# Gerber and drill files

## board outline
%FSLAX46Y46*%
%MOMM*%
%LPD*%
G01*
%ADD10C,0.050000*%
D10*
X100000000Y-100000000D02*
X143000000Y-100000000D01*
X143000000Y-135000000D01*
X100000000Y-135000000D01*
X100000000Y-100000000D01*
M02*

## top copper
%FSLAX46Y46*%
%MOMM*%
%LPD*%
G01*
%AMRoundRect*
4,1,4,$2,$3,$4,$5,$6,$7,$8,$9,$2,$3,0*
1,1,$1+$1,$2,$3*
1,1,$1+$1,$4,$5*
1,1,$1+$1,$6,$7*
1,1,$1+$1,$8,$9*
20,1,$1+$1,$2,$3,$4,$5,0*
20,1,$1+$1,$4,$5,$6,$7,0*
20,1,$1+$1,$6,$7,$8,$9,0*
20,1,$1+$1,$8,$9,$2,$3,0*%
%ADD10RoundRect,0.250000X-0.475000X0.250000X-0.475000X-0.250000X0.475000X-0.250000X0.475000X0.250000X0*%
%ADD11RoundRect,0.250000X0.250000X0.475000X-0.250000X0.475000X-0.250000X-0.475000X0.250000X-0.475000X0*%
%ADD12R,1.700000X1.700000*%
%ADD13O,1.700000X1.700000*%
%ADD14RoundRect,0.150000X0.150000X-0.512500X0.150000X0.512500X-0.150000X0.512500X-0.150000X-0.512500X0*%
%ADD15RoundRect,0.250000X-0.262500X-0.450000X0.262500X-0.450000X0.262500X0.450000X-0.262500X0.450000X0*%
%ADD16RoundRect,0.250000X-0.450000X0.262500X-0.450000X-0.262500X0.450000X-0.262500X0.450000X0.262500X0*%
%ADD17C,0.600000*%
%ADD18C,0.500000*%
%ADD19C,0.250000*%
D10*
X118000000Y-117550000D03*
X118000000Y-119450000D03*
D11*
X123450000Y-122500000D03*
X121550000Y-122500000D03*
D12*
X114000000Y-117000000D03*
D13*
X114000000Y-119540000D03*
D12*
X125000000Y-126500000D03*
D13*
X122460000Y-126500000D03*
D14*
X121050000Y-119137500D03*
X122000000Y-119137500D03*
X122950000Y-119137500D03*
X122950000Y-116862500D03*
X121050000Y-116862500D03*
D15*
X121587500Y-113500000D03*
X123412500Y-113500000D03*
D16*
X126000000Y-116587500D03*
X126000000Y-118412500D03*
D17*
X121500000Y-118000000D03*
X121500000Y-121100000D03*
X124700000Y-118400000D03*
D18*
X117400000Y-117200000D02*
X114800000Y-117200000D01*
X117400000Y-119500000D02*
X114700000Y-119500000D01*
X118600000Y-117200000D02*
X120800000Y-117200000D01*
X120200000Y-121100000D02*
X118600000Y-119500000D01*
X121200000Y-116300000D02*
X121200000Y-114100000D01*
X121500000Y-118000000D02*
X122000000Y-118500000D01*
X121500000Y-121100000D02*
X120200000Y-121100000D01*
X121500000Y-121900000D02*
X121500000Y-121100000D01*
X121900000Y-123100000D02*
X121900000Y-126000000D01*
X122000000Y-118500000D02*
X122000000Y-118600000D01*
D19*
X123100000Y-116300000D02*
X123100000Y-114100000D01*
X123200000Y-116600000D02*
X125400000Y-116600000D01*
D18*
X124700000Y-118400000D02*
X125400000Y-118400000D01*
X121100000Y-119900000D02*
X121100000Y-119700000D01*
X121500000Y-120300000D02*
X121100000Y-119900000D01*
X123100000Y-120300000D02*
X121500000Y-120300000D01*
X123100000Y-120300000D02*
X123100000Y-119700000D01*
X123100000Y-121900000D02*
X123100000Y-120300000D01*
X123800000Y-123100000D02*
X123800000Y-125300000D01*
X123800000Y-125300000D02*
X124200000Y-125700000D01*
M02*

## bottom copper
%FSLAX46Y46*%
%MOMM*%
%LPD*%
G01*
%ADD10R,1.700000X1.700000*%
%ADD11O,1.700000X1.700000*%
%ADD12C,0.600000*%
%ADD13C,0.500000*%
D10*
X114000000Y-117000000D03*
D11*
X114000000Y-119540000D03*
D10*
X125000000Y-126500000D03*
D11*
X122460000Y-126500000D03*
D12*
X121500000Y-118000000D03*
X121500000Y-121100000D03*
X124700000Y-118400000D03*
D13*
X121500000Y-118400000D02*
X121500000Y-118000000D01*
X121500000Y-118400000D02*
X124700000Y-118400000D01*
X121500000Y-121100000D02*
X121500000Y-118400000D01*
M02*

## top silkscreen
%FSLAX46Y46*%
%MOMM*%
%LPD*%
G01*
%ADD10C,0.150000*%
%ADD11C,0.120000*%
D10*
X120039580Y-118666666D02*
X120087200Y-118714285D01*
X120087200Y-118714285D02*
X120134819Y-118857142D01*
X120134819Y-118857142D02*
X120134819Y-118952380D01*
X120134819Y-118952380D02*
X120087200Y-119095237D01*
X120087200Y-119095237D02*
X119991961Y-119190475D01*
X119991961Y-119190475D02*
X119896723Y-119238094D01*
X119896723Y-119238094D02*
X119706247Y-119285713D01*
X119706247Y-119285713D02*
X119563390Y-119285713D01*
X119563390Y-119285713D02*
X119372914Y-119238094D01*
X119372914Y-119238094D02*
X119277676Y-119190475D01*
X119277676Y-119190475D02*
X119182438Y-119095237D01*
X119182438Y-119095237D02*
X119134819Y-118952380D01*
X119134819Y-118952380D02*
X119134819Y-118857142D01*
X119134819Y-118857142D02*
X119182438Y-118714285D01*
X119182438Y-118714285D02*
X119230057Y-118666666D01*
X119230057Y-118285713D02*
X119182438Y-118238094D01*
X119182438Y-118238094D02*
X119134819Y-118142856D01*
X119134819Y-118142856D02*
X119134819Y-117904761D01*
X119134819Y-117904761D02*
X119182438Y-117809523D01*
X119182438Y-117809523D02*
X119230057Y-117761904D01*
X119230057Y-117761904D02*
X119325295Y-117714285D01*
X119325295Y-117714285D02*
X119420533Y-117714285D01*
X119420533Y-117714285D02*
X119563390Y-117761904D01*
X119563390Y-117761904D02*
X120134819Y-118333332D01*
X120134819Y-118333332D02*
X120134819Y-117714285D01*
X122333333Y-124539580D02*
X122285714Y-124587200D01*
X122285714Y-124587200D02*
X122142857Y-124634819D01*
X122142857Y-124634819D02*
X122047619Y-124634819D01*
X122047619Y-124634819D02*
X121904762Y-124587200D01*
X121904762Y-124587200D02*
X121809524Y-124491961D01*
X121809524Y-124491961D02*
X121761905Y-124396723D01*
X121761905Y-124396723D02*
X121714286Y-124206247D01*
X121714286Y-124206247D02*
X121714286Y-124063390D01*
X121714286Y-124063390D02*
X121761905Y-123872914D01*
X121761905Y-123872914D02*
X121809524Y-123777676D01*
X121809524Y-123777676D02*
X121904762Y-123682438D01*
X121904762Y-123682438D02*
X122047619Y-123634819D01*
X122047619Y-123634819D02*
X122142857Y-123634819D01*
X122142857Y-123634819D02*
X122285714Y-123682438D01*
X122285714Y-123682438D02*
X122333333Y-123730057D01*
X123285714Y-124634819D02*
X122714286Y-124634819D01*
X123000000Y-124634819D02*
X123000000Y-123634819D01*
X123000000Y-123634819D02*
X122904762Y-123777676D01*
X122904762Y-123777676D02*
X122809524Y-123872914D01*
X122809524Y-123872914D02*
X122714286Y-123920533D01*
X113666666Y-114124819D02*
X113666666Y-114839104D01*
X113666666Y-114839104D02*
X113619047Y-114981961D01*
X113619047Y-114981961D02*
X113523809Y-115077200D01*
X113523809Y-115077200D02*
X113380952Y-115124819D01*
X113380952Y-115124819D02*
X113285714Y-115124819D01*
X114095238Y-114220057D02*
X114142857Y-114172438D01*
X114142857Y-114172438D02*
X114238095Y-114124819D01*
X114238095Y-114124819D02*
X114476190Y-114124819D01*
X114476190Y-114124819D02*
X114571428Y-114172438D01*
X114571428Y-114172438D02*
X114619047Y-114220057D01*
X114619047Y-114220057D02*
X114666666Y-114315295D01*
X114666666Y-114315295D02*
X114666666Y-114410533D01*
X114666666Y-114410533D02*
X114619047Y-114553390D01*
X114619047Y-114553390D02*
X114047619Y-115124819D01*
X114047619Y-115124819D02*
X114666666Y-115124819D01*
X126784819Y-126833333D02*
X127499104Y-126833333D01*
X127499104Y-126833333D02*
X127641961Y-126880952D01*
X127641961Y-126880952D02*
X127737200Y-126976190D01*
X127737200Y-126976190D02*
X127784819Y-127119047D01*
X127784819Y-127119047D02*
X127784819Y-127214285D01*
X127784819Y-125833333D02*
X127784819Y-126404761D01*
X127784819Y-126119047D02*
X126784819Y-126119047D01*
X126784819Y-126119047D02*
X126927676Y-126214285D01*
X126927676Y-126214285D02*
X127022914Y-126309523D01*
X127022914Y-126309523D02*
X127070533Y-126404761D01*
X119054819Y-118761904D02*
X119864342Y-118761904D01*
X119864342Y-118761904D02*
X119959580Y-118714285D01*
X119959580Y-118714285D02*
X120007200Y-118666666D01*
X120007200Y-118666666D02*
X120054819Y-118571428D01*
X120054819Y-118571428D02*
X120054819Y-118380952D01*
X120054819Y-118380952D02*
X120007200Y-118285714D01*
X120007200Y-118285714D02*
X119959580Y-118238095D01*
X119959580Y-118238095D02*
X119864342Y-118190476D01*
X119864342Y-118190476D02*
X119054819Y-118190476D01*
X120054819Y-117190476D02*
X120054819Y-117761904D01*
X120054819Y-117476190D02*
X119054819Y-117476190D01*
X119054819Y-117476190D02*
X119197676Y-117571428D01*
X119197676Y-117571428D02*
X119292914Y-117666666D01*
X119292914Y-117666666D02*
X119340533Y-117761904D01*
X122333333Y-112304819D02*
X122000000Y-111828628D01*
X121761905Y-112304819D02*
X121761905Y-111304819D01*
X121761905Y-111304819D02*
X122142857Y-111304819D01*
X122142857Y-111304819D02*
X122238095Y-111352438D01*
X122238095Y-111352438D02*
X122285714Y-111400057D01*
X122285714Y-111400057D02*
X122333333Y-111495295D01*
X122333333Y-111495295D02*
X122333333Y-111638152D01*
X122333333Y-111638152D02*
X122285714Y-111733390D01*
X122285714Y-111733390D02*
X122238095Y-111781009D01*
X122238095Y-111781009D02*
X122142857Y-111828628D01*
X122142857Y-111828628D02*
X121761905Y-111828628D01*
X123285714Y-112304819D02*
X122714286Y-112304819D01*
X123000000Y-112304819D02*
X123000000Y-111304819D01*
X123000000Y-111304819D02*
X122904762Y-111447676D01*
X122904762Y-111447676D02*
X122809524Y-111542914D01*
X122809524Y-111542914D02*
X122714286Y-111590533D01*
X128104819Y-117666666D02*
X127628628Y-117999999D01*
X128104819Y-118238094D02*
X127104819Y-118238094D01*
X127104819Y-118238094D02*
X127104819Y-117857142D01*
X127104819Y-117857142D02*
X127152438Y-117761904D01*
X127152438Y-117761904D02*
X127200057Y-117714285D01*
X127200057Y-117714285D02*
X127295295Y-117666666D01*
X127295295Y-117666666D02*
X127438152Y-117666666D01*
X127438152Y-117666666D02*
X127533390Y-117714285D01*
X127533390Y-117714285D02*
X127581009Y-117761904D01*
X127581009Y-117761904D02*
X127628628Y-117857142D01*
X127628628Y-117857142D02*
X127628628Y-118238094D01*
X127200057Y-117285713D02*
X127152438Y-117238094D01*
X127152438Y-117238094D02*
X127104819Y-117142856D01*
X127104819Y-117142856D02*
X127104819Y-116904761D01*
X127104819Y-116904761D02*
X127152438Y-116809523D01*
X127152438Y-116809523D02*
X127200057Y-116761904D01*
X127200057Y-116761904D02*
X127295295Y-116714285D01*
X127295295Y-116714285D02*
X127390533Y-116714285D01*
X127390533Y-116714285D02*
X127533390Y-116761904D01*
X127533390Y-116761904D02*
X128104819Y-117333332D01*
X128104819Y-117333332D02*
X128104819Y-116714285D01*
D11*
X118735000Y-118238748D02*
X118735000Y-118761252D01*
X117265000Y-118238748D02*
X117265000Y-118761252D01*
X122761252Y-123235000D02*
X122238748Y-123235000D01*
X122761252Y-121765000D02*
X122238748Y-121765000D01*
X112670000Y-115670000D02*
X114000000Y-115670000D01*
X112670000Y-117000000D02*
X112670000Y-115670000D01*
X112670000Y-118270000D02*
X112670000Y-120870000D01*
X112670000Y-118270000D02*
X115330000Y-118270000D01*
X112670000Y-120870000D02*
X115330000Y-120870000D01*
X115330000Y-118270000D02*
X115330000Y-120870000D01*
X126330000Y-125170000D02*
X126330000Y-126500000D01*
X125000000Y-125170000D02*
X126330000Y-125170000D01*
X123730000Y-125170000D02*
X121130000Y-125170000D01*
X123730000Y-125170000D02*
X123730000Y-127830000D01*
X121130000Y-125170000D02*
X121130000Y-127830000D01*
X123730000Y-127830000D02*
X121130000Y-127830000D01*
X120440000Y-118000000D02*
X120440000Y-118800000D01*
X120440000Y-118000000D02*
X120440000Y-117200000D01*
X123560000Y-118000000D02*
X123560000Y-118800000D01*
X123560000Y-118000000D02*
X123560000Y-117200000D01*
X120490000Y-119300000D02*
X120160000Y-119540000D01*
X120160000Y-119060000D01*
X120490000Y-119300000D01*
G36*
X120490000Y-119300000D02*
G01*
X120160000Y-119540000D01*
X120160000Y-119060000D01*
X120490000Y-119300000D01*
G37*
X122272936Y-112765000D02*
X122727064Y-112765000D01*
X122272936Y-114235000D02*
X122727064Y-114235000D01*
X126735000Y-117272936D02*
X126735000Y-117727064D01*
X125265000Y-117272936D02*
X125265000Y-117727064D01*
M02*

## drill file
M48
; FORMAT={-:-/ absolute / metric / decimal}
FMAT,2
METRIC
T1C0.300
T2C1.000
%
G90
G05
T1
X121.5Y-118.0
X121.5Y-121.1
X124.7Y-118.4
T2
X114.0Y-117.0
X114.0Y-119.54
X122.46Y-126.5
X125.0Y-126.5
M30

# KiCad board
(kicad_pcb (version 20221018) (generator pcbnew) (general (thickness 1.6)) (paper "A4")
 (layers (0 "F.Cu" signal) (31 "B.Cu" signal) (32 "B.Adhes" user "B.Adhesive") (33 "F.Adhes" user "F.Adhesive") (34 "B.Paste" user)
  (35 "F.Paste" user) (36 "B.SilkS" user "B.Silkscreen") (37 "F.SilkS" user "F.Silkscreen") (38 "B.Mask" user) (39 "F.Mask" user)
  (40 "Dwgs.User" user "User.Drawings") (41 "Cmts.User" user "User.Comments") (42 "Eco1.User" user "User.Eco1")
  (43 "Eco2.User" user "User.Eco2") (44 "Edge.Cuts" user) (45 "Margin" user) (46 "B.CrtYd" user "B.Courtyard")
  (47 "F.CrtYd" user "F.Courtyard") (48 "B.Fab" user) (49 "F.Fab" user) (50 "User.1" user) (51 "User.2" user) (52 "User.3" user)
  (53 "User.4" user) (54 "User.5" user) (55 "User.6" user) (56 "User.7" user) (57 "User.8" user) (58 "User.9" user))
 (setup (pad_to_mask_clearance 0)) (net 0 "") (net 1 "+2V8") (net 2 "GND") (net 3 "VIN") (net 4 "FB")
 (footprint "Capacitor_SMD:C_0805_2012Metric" (layer "F.Cu") (at 118 118.5 -90)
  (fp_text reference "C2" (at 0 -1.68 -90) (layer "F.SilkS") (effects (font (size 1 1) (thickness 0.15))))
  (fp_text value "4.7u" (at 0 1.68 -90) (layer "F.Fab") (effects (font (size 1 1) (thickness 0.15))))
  (fp_line (start -0.261252 -0.735) (end 0.261252 -0.735) (stroke (width 0.12) (type solid)) (layer "F.SilkS"))
  (fp_line (start -0.261252 0.735) (end 0.261252 0.735) (stroke (width 0.12) (type solid)) (layer "F.SilkS"))
  (pad "1" smd roundrect (at -0.95 0 270) (size 1 1.45) (layers "F.Cu" "F.Paste" "F.Mask") (roundrect_rratio 0.25) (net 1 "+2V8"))
  (pad "2" smd roundrect (at 0.95 0 270) (size 1 1.45) (layers "F.Cu" "F.Paste" "F.Mask") (roundrect_rratio 0.25) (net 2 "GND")))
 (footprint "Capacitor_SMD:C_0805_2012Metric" (layer "F.Cu") (at 122.5 122.5 180)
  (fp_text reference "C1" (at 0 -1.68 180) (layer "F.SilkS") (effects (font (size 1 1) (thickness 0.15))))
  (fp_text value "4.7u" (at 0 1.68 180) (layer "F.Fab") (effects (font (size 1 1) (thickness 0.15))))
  (fp_line (start -0.261252 -0.735) (end 0.261252 -0.735) (stroke (width 0.12) (type solid)) (layer "F.SilkS"))
  (fp_line (start -0.261252 0.735) (end 0.261252 0.735) (stroke (width 0.12) (type solid)) (layer "F.SilkS"))
  (pad "1" smd roundrect (at -0.95 0 180) (size 1 1.45) (layers "F.Cu" "F.Paste" "F.Mask") (roundrect_rratio 0.25) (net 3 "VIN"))
  (pad "2" smd roundrect (at 0.95 0 180) (size 1 1.45) (layers "F.Cu" "F.Paste" "F.Mask") (roundrect_rratio 0.25) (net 2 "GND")))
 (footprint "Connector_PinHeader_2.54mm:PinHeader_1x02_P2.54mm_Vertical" (layer "F.Cu") (at 114 117)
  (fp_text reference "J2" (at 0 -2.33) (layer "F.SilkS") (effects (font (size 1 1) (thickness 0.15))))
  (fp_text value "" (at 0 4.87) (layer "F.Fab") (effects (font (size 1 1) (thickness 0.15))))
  (fp_line (start -1.33 -1.33) (end 0 -1.33) (stroke (width 0.12) (type solid)) (layer "F.SilkS"))
  (fp_line (start -1.33 0) (end -1.33 -1.33) (stroke (width 0.12) (type solid)) (layer "F.SilkS"))
  (fp_line (start -1.33 1.27) (end -1.33 3.87) (stroke (width 0.12) (type solid)) (layer "F.SilkS"))
  (fp_line (start -1.33 1.27) (end 1.33 1.27) (stroke (width 0.12) (type solid)) (layer "F.SilkS"))
  (fp_line (start -1.33 3.87) (end 1.33 3.87) (stroke (width 0.12) (type solid)) (layer "F.SilkS"))
  (fp_line (start 1.33 1.27) (end 1.33 3.87) (stroke (width 0.12) (type solid)) (layer "F.SilkS"))
  (pad "1" thru_hole rect (at 0 0) (size 1.7 1.7) (drill 1) (layers "*.Cu" "*.Mask") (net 1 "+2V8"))
  (pad "2" thru_hole oval (at 0 2.54) (size 1.7 1.7) (drill 1) (layers "*.Cu" "*.Mask") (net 2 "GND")))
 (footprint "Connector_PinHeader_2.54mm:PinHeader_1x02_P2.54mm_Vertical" (layer "F.Cu") (at 125 126.5 -90)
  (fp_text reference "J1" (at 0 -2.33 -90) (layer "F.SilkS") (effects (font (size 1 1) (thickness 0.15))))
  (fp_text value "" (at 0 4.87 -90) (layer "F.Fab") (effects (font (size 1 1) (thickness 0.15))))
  (fp_line (start -1.33 -1.33) (end 0 -1.33) (stroke (width 0.12) (type solid)) (layer "F.SilkS"))
  (fp_line (start -1.33 0) (end -1.33 -1.33) (stroke (width 0.12) (type solid)) (layer "F.SilkS"))
  (fp_line (start -1.33 1.27) (end -1.33 3.87) (stroke (width 0.12) (type solid)) (layer "F.SilkS"))
  (fp_line (start -1.33 1.27) (end 1.33 1.27) (stroke (width 0.12) (type solid)) (layer "F.SilkS"))
  (fp_line (start -1.33 3.87) (end 1.33 3.87) (stroke (width 0.12) (type solid)) (layer "F.SilkS"))
  (fp_line (start 1.33 1.27) (end 1.33 3.87) (stroke (width 0.12) (type solid)) (layer "F.SilkS"))
  (pad "1" thru_hole rect (at 0 0 270) (size 1.7 1.7) (drill 1) (layers "*.Cu" "*.Mask") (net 3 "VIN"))
  (pad "2" thru_hole oval (at 0 2.54 270) (size 1.7 1.7) (drill 1) (layers "*.Cu" "*.Mask") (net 2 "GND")))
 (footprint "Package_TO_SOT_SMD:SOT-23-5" (layer "F.Cu") (at 122 118 90)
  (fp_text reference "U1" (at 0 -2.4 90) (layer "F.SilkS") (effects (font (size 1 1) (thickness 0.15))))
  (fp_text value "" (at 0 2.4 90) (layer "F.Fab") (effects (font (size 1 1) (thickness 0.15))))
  (fp_line (start 0 -1.56) (end -0.8 -1.56) (stroke (width 0.12) (type solid)) (layer "F.SilkS"))
  (fp_line (start 0 -1.56) (end 0.8 -1.56) (stroke (width 0.12) (type solid)) (layer "F.SilkS"))
  (fp_line (start 0 1.56) (end -0.8 1.56) (stroke (width 0.12) (type solid)) (layer "F.SilkS"))
  (fp_line (start 0 1.56) (end 0.8 1.56) (stroke (width 0.12) (type solid)) (layer "F.SilkS"))
  (fp_poly
   (pts (xy -1.3 -1.51) (xy -1.54 -1.84) (xy -1.06 -1.84) (xy -1.3 -1.51)) (stroke (width 0.12) (type solid)) (fill solid) (layer "F.SilkS"))
  (pad "1" smd roundrect (at -1.1375 -0.95 90) (size 1.325 0.6) (layers "F.Cu" "F.Paste" "F.Mask") (roundrect_rratio 0.25) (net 3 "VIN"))
  (pad "2" smd roundrect (at -1.1375 0 90) (size 1.325 0.6) (layers "F.Cu" "F.Paste" "F.Mask") (roundrect_rratio 0.25) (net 2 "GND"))
  (pad "3" smd roundrect (at -1.1375 0.95 90) (size 1.325 0.6) (layers "F.Cu" "F.Paste" "F.Mask") (roundrect_rratio 0.25) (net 3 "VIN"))
  (pad "4" smd roundrect (at 1.1375 0.95 90) (size 1.325 0.6) (layers "F.Cu" "F.Paste" "F.Mask") (roundrect_rratio 0.25) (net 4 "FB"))
  (pad "5" smd roundrect (at 1.1375 -0.95 90) (size 1.325 0.6) (layers "F.Cu" "F.Paste" "F.Mask") (roundrect_rratio 0.25) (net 1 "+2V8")))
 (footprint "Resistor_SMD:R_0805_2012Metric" (layer "F.Cu") (at 122.5 113.5)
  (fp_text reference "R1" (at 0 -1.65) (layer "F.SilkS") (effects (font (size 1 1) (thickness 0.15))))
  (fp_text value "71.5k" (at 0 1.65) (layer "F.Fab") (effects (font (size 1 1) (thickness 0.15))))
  (fp_line (start -0.227064 -0.735) (end 0.227064 -0.735) (stroke (width 0.12) (type solid)) (layer "F.SilkS"))
  (fp_line (start -0.227064 0.735) (end 0.227064 0.735) (stroke (width 0.12) (type solid)) (layer "F.SilkS"))
  (pad "1" smd roundrect (at -0.9125 0) (size 1.025 1.4) (layers "F.Cu" "F.Paste" "F.Mask") (roundrect_rratio 0.243902) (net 1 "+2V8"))
  (pad "2" smd roundrect (at 0.9125 0) (size 1.025 1.4) (layers "F.Cu" "F.Paste" "F.Mask") (roundrect_rratio 0.243902) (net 4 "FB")))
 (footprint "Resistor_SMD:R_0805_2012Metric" (layer "F.Cu") (at 126 117.5 -90)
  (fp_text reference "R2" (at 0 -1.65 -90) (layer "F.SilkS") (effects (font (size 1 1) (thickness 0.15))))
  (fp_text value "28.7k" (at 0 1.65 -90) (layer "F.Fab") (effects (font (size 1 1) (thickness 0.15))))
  (fp_line (start -0.227064 -0.735) (end 0.227064 -0.735) (stroke (width 0.12) (type solid)) (layer "F.SilkS"))
  (fp_line (start -0.227064 0.735) (end 0.227064 0.735) (stroke (width 0.12) (type solid)) (layer "F.SilkS"))
  (pad "1" smd roundrect (at -0.9125 0 270) (size 1.025 1.4) (layers "F.Cu" "F.Paste" "F.Mask") (roundrect_rratio 0.243902) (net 4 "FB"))
  (pad "2" smd roundrect (at 0.9125 0 270) (size 1.025 1.4) (layers "F.Cu" "F.Paste" "F.Mask") (roundrect_rratio 0.243902) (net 2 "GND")))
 (gr_rect (start 100 100) (end 143 135) (stroke (width 0.05) (type default)) (fill none) (layer "Edge.Cuts"))
 (segment (start 117.4 117.2) (end 114.8 117.2) (width 0.5) (layer "F.Cu") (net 1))
 (segment (start 117.4 119.5) (end 114.7 119.5) (width 0.5) (layer "F.Cu") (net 2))
 (segment (start 118.6 117.2) (end 120.8 117.2) (width 0.5) (layer "F.Cu") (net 1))
 (segment (start 120.2 121.1) (end 118.6 119.5) (width 0.5) (layer "F.Cu") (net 2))
 (segment (start 121.2 116.3) (end 121.2 114.1) (width 0.5) (layer "F.Cu") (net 1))
 (segment (start 121.5 118) (end 122 118.5) (width 0.5) (layer "F.Cu") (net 2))
 (segment (start 121.5 121.1) (end 120.2 121.1) (width 0.5) (layer "F.Cu") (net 2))
 (segment (start 121.5 121.9) (end 121.5 121.1) (width 0.5) (layer "F.Cu") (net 2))
 (segment (start 121.9 123.1) (end 121.9 126) (width 0.5) (layer "F.Cu") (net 2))
 (segment (start 122 118.5) (end 122 118.6) (width 0.5) (layer "F.Cu") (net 2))
 (segment (start 123.1 116.3) (end 123.1 114.1) (width 0.25) (layer "F.Cu") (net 4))
 (segment (start 123.2 116.6) (end 125.4 116.6) (width 0.25) (layer "F.Cu") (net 4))
 (segment (start 124.7 118.4) (end 125.4 118.4) (width 0.5) (layer "F.Cu") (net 2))
 (via (at 121.5 118) (size 0.6) (drill 0.3) (layers "F.Cu" "B.Cu") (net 2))
 (via (at 121.5 121.1) (size 0.6) (drill 0.3) (layers "F.Cu" "B.Cu") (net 2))
 (via (at 124.7 118.4) (size 0.6) (drill 0.3) (layers "F.Cu" "B.Cu") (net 2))
 (segment (start 121.1 119.9) (end 121.1 119.7) (width 0.5) (layer "F.Cu") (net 3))
 (segment (start 121.5 118.4) (end 121.5 118) (width 0.5) (layer "B.Cu") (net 2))
 (segment (start 121.5 118.4) (end 124.7 118.4) (width 0.5) (layer "B.Cu") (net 2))
 (segment (start 121.5 120.3) (end 121.1 119.9) (width 0.5) (layer "F.Cu") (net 3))
 (segment (start 121.5 121.1) (end 121.5 118.4) (width 0.5) (layer "B.Cu") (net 2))
 (segment (start 123.1 120.3) (end 121.5 120.3) (width 0.5) (layer "F.Cu") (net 3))
 (segment (start 123.1 120.3) (end 123.1 119.7) (width 0.5) (layer "F.Cu") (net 3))
 (segment (start 123.1 121.9) (end 123.1 120.3) (width 0.5) (layer "F.Cu") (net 3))
 (segment (start 123.8 123.1) (end 123.8 125.3) (width 0.5) (layer "F.Cu") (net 3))
 (segment (start 123.8 125.3) (end 124.2 125.7) (width 0.5) (layer "F.Cu") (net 3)))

